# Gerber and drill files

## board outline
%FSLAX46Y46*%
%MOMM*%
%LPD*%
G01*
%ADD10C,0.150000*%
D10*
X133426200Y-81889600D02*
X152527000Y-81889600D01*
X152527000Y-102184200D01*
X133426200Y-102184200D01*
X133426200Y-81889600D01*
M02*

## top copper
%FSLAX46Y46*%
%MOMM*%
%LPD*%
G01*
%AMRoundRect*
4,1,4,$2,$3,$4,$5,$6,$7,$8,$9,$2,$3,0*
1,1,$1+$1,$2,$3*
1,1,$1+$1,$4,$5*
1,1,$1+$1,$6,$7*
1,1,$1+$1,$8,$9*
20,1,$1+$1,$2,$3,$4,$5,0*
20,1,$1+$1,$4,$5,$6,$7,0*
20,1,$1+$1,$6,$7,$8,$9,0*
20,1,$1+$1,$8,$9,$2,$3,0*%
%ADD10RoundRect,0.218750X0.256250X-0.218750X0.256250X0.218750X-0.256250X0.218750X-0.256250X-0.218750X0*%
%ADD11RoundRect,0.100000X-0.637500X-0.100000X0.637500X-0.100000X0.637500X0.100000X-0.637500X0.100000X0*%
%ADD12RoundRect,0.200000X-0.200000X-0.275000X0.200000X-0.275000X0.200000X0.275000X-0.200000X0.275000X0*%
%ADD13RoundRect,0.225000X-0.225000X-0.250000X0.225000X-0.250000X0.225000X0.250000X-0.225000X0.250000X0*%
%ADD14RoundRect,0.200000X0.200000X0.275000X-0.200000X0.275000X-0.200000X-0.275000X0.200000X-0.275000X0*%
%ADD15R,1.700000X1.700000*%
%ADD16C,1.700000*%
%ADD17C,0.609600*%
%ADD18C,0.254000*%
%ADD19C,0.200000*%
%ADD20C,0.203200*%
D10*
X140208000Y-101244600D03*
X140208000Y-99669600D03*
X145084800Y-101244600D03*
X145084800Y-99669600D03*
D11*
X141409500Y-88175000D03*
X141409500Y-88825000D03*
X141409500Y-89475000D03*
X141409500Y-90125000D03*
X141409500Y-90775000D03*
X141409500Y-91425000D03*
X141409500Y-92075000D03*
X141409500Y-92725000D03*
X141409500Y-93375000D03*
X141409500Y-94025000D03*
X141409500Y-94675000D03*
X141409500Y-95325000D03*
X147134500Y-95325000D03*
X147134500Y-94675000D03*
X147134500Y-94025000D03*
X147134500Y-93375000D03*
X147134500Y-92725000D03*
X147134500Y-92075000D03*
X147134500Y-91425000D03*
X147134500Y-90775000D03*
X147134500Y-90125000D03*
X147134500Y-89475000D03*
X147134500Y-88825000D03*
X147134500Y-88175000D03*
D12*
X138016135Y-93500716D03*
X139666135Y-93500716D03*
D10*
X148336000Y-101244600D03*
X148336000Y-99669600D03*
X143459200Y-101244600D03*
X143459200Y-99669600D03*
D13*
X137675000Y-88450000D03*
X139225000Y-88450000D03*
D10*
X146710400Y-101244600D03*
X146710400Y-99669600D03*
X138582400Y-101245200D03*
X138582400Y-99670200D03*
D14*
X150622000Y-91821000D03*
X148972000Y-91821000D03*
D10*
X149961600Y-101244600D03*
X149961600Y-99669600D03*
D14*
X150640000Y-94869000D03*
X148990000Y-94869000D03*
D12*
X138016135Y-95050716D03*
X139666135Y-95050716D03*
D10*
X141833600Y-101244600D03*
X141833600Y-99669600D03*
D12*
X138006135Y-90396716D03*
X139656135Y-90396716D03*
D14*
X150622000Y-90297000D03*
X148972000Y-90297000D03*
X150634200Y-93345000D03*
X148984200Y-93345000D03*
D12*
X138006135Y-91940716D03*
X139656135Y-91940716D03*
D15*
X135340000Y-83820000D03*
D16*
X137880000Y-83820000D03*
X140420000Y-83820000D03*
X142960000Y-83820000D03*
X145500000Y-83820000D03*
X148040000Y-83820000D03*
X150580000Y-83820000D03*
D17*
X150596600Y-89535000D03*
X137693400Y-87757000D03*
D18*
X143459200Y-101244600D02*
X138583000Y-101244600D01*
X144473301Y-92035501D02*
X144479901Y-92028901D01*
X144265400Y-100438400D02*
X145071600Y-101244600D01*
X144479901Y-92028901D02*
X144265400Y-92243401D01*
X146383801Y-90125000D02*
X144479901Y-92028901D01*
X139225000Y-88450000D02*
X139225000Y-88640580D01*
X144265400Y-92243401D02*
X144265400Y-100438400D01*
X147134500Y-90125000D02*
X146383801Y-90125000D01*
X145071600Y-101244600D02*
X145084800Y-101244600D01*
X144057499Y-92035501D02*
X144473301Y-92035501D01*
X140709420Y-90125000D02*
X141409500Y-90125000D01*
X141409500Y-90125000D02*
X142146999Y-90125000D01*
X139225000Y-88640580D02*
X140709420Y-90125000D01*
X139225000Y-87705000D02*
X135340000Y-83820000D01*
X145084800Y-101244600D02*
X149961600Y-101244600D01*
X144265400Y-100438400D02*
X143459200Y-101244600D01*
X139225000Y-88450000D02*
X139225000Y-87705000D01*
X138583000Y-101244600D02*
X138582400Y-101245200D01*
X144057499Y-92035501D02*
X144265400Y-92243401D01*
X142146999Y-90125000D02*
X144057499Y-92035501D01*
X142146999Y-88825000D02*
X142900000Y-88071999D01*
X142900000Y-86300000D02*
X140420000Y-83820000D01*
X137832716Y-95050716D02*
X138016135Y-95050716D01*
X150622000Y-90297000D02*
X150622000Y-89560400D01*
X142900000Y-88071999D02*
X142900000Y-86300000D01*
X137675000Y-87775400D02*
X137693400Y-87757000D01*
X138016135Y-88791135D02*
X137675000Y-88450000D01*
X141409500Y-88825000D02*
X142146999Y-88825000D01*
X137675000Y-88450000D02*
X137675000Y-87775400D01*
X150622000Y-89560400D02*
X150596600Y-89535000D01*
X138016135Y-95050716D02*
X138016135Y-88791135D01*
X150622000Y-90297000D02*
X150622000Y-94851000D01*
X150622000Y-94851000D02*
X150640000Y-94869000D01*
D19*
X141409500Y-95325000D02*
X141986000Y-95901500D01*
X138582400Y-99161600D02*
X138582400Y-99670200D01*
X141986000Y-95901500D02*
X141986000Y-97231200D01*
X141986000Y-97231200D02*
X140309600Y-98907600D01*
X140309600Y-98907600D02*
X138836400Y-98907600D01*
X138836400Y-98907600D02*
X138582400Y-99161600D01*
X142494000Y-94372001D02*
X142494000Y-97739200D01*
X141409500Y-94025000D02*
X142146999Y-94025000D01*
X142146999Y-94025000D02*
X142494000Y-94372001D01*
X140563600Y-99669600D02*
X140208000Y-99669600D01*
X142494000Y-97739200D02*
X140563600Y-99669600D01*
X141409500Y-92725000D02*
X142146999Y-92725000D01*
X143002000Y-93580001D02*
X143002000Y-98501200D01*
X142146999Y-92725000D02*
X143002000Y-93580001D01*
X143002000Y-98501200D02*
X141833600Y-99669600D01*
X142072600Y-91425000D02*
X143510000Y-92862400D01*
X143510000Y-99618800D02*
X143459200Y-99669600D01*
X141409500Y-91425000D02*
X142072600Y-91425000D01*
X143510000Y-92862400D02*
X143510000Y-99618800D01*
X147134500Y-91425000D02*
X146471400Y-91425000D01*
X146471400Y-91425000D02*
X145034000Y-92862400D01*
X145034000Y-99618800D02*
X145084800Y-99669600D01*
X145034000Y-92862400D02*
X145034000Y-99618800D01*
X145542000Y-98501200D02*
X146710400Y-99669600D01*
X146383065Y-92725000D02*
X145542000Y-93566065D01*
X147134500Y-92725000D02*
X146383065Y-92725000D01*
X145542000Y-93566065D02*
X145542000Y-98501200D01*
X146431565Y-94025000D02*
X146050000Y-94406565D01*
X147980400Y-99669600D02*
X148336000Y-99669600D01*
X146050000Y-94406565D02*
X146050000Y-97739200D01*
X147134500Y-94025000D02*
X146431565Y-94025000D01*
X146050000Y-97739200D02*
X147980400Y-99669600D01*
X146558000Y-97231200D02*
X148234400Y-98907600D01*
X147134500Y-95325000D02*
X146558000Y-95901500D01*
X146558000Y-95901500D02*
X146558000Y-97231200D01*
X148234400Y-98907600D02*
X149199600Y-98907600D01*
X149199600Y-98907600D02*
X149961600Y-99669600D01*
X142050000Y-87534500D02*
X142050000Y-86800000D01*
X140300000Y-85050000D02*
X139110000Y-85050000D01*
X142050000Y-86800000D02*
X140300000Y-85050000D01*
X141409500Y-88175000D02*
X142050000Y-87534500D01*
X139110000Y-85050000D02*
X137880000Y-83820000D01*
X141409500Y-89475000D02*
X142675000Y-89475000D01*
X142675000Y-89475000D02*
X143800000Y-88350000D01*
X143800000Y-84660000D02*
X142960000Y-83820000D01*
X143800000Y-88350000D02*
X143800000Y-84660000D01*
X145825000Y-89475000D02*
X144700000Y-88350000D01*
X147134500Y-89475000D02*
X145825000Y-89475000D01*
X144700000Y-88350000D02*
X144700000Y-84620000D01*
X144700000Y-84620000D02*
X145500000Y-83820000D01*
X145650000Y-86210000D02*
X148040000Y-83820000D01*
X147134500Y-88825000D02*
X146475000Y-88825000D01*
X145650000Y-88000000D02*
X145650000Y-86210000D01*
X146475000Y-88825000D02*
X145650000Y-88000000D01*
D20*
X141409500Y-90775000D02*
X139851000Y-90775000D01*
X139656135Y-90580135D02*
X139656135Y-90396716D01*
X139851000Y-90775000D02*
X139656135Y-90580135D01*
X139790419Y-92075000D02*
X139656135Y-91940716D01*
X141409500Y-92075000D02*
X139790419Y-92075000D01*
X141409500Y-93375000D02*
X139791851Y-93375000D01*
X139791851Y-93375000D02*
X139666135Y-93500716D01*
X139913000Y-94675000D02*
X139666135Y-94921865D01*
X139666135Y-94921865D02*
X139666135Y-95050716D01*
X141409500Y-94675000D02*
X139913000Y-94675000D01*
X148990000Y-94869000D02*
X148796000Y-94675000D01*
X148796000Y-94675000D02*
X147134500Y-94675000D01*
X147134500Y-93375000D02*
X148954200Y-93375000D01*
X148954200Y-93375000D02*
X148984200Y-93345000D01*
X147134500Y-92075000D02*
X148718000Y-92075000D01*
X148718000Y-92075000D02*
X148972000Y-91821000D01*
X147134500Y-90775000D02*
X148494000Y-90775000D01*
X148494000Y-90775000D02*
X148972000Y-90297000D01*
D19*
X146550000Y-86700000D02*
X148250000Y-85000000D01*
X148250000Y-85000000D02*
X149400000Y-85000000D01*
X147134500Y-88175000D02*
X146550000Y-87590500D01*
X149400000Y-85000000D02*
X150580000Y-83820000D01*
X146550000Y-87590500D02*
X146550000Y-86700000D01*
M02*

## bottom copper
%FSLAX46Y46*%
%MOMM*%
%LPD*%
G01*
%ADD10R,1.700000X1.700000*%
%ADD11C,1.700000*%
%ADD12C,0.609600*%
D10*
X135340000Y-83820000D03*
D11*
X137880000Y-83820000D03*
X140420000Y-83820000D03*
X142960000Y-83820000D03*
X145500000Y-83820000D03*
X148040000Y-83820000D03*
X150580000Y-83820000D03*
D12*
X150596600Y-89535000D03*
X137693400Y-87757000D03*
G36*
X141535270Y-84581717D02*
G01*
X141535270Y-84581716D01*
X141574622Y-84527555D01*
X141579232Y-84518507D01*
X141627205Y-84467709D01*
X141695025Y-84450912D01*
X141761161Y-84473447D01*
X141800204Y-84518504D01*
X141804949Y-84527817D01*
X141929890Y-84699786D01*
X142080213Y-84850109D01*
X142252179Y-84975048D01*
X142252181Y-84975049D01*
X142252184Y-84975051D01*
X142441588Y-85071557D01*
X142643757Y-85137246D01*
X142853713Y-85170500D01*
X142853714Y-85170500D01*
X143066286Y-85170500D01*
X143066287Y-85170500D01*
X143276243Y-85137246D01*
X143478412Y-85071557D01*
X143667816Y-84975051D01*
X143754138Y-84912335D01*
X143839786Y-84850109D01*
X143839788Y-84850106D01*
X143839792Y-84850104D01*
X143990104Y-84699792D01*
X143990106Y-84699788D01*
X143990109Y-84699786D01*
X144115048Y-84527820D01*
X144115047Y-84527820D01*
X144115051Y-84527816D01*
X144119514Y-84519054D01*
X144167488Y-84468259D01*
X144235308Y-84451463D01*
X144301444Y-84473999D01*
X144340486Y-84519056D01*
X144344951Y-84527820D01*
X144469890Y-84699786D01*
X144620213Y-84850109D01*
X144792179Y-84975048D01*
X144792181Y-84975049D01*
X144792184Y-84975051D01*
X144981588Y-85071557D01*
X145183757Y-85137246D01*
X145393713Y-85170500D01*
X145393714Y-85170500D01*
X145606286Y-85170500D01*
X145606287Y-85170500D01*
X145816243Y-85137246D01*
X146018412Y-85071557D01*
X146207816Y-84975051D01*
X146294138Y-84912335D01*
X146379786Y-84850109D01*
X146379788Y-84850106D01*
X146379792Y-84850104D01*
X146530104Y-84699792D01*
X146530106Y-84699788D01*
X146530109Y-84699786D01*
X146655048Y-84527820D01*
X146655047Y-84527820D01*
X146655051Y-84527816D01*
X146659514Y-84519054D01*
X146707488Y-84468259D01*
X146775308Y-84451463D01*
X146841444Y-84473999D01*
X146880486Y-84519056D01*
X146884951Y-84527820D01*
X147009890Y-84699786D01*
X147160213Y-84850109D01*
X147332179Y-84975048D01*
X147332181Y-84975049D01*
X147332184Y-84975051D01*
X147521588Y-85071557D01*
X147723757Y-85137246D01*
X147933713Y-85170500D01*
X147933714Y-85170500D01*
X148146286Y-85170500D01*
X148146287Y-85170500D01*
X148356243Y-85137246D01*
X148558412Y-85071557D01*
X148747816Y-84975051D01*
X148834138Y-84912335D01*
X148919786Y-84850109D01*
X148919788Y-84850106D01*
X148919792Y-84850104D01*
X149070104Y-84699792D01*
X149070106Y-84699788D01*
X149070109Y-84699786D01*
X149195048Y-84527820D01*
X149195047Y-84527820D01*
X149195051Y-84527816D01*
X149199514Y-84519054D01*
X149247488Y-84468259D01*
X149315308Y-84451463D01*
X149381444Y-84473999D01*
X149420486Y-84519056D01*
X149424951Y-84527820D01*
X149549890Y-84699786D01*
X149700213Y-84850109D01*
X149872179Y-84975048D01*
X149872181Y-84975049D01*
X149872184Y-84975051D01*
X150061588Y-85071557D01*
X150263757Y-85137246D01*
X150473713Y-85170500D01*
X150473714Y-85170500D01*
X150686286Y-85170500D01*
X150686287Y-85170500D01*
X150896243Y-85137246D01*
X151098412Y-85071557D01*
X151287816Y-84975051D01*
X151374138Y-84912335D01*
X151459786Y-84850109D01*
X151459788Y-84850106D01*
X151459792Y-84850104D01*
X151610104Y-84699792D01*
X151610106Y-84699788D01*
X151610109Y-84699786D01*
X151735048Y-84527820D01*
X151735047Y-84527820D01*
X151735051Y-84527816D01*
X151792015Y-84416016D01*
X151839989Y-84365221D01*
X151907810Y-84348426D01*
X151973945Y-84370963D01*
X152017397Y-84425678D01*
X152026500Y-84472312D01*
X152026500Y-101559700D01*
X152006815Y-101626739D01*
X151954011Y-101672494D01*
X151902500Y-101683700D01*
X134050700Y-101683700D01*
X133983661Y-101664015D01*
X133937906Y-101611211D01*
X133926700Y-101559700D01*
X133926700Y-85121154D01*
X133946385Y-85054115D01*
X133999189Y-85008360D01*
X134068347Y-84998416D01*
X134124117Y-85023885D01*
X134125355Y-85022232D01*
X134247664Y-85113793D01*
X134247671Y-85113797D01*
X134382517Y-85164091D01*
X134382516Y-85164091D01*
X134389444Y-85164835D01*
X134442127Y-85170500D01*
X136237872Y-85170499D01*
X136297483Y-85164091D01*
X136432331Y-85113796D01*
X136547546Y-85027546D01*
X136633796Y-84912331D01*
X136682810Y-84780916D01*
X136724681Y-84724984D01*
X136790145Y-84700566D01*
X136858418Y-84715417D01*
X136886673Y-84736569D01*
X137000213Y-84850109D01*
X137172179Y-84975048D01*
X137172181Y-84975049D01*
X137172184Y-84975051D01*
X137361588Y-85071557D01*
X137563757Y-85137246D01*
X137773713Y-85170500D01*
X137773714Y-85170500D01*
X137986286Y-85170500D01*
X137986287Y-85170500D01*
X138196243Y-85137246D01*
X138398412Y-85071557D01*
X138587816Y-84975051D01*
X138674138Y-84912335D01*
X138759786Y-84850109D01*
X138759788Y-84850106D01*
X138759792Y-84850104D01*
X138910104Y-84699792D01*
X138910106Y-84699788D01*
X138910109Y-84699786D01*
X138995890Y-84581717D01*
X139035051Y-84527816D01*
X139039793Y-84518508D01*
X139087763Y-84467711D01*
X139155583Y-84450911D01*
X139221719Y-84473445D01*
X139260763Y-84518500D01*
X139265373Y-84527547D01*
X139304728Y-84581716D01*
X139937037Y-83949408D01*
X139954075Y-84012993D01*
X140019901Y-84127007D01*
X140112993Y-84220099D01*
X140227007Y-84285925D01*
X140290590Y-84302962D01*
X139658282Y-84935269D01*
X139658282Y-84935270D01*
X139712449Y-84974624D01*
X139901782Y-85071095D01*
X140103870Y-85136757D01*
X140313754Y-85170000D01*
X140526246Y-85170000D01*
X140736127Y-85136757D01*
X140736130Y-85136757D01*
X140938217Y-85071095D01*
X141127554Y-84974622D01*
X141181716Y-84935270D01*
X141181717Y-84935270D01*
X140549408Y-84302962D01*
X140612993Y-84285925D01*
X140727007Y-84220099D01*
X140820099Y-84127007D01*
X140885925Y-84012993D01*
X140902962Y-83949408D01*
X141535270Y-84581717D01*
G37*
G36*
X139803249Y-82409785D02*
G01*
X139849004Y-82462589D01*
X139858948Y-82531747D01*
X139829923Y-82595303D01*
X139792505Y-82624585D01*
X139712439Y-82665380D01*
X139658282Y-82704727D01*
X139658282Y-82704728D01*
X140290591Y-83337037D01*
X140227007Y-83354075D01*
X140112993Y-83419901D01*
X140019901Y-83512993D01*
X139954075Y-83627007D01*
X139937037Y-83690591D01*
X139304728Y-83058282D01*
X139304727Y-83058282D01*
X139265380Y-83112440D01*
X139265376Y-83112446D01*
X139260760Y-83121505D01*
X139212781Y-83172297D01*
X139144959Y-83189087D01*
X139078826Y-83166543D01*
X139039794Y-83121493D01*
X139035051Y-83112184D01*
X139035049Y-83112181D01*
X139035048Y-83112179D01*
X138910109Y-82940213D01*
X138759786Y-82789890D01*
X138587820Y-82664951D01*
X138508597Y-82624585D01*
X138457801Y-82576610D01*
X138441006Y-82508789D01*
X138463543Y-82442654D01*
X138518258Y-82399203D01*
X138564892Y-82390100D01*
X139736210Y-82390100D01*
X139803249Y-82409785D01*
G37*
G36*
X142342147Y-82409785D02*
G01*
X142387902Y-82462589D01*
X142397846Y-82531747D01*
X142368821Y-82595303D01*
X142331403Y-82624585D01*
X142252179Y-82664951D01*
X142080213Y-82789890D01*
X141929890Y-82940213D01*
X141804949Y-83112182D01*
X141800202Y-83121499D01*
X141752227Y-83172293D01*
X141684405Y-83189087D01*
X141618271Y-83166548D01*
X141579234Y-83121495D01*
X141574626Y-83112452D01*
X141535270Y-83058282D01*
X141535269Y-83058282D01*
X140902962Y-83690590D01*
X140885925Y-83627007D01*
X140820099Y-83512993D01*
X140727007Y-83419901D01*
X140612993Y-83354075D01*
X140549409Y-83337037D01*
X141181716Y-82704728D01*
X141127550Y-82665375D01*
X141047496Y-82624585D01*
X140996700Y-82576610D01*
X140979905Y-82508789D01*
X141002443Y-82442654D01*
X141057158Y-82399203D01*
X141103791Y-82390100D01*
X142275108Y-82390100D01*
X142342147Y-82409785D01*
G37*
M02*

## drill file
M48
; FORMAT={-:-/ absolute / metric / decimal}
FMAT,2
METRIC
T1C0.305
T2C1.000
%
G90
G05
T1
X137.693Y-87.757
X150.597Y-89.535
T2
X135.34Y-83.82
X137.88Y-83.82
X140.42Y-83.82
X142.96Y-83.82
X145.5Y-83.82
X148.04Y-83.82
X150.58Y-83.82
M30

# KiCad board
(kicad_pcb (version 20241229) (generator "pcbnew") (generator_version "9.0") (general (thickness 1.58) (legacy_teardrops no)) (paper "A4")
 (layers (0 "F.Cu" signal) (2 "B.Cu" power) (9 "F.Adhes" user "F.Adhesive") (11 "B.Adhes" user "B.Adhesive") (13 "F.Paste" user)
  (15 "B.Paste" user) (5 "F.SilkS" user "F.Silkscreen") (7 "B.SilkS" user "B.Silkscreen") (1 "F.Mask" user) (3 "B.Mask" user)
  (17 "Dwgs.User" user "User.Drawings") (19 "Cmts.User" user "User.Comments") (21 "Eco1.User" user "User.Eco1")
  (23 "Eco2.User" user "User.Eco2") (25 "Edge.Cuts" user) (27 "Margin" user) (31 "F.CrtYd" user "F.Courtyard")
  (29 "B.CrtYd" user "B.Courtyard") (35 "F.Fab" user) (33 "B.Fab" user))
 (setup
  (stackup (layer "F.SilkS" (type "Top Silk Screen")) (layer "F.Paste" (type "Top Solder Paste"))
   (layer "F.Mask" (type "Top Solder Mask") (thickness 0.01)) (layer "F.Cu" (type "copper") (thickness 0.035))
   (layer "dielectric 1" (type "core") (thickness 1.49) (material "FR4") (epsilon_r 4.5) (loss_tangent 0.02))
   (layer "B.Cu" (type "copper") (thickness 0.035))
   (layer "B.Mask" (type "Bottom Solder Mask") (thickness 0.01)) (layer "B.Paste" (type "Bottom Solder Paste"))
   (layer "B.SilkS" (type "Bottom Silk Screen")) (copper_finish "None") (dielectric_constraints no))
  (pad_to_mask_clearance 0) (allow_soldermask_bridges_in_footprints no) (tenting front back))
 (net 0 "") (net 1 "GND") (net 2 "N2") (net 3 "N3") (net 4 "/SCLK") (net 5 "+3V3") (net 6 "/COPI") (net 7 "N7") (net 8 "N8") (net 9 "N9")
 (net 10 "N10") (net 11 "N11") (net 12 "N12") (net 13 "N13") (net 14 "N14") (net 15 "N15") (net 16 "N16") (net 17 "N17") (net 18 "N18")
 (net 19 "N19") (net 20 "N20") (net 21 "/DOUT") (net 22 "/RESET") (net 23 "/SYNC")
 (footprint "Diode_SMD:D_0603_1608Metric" (layer "F.Cu") (at 140.208 100.4571 90)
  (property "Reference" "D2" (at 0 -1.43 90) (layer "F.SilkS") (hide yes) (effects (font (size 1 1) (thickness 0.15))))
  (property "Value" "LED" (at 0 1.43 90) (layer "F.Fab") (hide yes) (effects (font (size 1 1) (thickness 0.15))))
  (pad "1" smd roundrect (at -0.7875 0 90) (size 0.875 0.95) (layers "F.Cu" "F.Mask" "F.Paste") (roundrect_rratio 0.25) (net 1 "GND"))
  (pad "2" smd roundrect (at 0.7875 0 90) (size 0.875 0.95) (layers "F.Cu" "F.Mask" "F.Paste") (roundrect_rratio 0.25) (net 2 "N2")))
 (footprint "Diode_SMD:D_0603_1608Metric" (layer "F.Cu") (at 145.0848 100.4571 90)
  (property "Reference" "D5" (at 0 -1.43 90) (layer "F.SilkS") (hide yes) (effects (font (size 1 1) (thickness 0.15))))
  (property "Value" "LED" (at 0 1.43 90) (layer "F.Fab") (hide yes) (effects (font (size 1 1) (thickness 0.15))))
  (pad "1" smd roundrect (at -0.7875 0 90) (size 0.875 0.95) (layers "F.Cu" "F.Mask" "F.Paste") (roundrect_rratio 0.25) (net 1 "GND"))
  (pad "2" smd roundrect (at 0.7875 0 90) (size 0.875 0.95) (layers "F.Cu" "F.Mask" "F.Paste") (roundrect_rratio 0.25) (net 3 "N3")))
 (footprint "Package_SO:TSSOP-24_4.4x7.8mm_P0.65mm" (layer "F.Cu") (at 144.272 91.75)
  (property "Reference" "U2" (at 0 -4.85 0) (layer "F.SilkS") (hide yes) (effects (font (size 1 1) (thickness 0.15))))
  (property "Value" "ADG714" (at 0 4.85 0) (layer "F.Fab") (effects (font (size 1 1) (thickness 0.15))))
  (pad "1" smd roundrect (at -2.8625 -3.575) (size 1.475 0.4) (layers "F.Cu" "F.Mask" "F.Paste") (roundrect_rratio 0.25) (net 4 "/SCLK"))
  (pad "2" smd roundrect (at -2.8625 -2.925) (size 1.475 0.4) (layers "F.Cu" "F.Mask" "F.Paste") (roundrect_rratio 0.25) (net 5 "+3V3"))
  (pad "3" smd roundrect (at -2.8625 -2.275) (size 1.475 0.4) (layers "F.Cu" "F.Mask" "F.Paste") (roundrect_rratio 0.25) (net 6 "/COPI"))
  (pad "4" smd roundrect (at -2.8625 -1.625) (size 1.475 0.4) (layers "F.Cu" "F.Mask" "F.Paste") (roundrect_rratio 0.25) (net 1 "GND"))
  (pad "5" smd roundrect (at -2.8625 -0.975) (size 1.475 0.4) (layers "F.Cu" "F.Mask" "F.Paste") (roundrect_rratio 0.25) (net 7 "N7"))
  (pad "6" smd roundrect (at -2.8625 -0.325) (size 1.475 0.4) (layers "F.Cu" "F.Mask" "F.Paste") (roundrect_rratio 0.25) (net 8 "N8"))
  (pad "7" smd roundrect (at -2.8625 0.325) (size 1.475 0.4) (layers "F.Cu" "F.Mask" "F.Paste") (roundrect_rratio 0.25) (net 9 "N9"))
  (pad "8" smd roundrect (at -2.8625 0.975) (size 1.475 0.4) (layers "F.Cu" "F.Mask" "F.Paste") (roundrect_rratio 0.25) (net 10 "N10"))
  (pad "9" smd roundrect (at -2.8625 1.625) (size 1.475 0.4) (layers "F.Cu" "F.Mask" "F.Paste") (roundrect_rratio 0.25) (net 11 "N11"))
  (pad "10" smd roundrect (at -2.8625 2.275) (size 1.475 0.4) (layers "F.Cu" "F.Mask" "F.Paste") (roundrect_rratio 0.25) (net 2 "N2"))
  (pad "11" smd roundrect (at -2.8625 2.925) (size 1.475 0.4) (layers "F.Cu" "F.Mask" "F.Paste") (roundrect_rratio 0.25) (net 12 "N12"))
  (pad "12" smd roundrect (at -2.8625 3.575) (size 1.475 0.4) (layers "F.Cu" "F.Mask" "F.Paste") (roundrect_rratio 0.25) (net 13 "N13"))
  (pad "13" smd roundrect (at 2.8625 3.575) (size 1.475 0.4) (layers "F.Cu" "F.Mask" "F.Paste") (roundrect_rratio 0.25) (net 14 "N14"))
  (pad "14" smd roundrect (at 2.8625 2.925) (size 1.475 0.4) (layers "F.Cu" "F.Mask" "F.Paste") (roundrect_rratio 0.25) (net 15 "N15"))
  (pad "15" smd roundrect (at 2.8625 2.275) (size 1.475 0.4) (layers "F.Cu" "F.Mask" "F.Paste") (roundrect_rratio 0.25) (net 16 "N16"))
  (pad "16" smd roundrect (at 2.8625 1.625) (size 1.475 0.4) (layers "F.Cu" "F.Mask" "F.Paste") (roundrect_rratio 0.25) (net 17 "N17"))
  (pad "17" smd roundrect (at 2.8625 0.975) (size 1.475 0.4) (layers "F.Cu" "F.Mask" "F.Paste") (roundrect_rratio 0.25) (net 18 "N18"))
  (pad "18" smd roundrect (at 2.8625 0.325) (size 1.475 0.4) (layers "F.Cu" "F.Mask" "F.Paste") (roundrect_rratio 0.25) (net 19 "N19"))
  (pad "19" smd roundrect (at 2.8625 -0.325) (size 1.475 0.4) (layers "F.Cu" "F.Mask" "F.Paste") (roundrect_rratio 0.25) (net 3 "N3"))
  (pad "20" smd roundrect (at 2.8625 -0.975) (size 1.475 0.4) (layers "F.Cu" "F.Mask" "F.Paste") (roundrect_rratio 0.25) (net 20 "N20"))
  (pad "21" smd roundrect (at 2.8625 -1.625) (size 1.475 0.4) (layers "F.Cu" "F.Mask" "F.Paste") (roundrect_rratio 0.25) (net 1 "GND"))
  (pad "22" smd roundrect (at 2.8625 -2.275) (size 1.475 0.4) (layers "F.Cu" "F.Mask" "F.Paste") (roundrect_rratio 0.25) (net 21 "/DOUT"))
  (pad "23" smd roundrect (at 2.8625 -2.925) (size 1.475 0.4) (layers "F.Cu" "F.Mask" "F.Paste") (roundrect_rratio 0.25) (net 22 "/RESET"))
  (pad "24" smd roundrect (at 2.8625 -3.575) (size 1.475 0.4) (layers "F.Cu" "F.Mask" "F.Paste") (roundrect_rratio 0.25) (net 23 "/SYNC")))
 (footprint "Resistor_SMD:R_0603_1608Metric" (layer "F.Cu") (at 138.841135 93.500716)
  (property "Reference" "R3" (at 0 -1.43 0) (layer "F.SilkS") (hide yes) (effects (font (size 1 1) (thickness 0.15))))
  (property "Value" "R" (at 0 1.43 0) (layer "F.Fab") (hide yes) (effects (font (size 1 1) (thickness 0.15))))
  (pad "1" smd roundrect (at -0.825 0) (size 0.8 0.95) (layers "F.Cu" "F.Mask" "F.Paste") (roundrect_rratio 0.25) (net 5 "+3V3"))
  (pad "2" smd roundrect (at 0.825 0) (size 0.8 0.95) (layers "F.Cu" "F.Mask" "F.Paste") (roundrect_rratio 0.25) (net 11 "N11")))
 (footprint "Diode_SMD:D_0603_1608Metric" (layer "F.Cu") (at 148.336 100.4571 90)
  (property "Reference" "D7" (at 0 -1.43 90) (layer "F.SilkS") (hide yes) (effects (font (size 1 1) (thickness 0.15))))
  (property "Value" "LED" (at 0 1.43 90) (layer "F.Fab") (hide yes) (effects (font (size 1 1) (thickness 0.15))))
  (pad "1" smd roundrect (at -0.7875 0 90) (size 0.875 0.95) (layers "F.Cu" "F.Mask" "F.Paste") (roundrect_rratio 0.25) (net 1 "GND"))
  (pad "2" smd roundrect (at 0.7875 0 90) (size 0.875 0.95) (layers "F.Cu" "F.Mask" "F.Paste") (roundrect_rratio 0.25) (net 16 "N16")))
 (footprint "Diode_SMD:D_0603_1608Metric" (layer "F.Cu") (at 143.4592 100.4571 90)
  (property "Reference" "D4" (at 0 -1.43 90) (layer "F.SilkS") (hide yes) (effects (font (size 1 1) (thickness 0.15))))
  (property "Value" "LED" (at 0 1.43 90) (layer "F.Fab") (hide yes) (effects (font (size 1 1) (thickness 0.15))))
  (pad "1" smd roundrect (at -0.7875 0 90) (size 0.875 0.95) (layers "F.Cu" "F.Mask" "F.Paste") (roundrect_rratio 0.25) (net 1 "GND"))
  (pad "2" smd roundrect (at 0.7875 0 90) (size 0.875 0.95) (layers "F.Cu" "F.Mask" "F.Paste") (roundrect_rratio 0.25) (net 8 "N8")))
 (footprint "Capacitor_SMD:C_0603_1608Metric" (layer "F.Cu") (at 138.45 88.45)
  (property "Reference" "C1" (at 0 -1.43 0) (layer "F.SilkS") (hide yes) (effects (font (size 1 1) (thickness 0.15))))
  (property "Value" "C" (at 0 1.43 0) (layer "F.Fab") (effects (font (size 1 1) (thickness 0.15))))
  (pad "1" smd roundrect (at -0.775 0) (size 0.9 0.95) (layers "F.Cu" "F.Mask" "F.Paste") (roundrect_rratio 0.25) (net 5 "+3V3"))
  (pad "2" smd roundrect (at 0.775 0) (size 0.9 0.95) (layers "F.Cu" "F.Mask" "F.Paste") (roundrect_rratio 0.25) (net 1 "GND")))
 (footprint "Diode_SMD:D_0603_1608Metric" (layer "F.Cu") (at 146.7104 100.4571 90)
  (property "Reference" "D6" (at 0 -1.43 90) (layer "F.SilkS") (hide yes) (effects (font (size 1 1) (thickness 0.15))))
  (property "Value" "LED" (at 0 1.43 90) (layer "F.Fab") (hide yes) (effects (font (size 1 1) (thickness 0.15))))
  (pad "1" smd roundrect (at -0.7875 0 90) (size 0.875 0.95) (layers "F.Cu" "F.Mask" "F.Paste") (roundrect_rratio 0.25) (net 1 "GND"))
  (pad "2" smd roundrect (at 0.7875 0 90) (size 0.875 0.95) (layers "F.Cu" "F.Mask" "F.Paste") (roundrect_rratio 0.25) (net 18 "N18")))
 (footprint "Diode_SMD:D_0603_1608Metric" (layer "F.Cu") (at 138.5824 100.4577 90)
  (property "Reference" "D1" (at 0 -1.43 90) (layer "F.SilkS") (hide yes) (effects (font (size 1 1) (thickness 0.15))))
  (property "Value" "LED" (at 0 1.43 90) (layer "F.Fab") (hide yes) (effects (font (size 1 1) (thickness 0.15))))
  (pad "1" smd roundrect (at -0.7875 0 90) (size 0.875 0.95) (layers "F.Cu" "F.Mask" "F.Paste") (roundrect_rratio 0.25) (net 1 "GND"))
  (pad "2" smd roundrect (at 0.7875 0 90) (size 0.875 0.95) (layers "F.Cu" "F.Mask" "F.Paste") (roundrect_rratio 0.25) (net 13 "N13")))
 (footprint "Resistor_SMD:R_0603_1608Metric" (layer "F.Cu") (at 149.797 91.821 180)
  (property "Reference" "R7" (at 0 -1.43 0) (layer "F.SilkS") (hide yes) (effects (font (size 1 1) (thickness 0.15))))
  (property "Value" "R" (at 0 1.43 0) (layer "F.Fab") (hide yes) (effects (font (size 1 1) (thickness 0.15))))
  (pad "1" smd roundrect (at -0.825 0 180) (size 0.8 0.95) (layers "F.Cu" "F.Mask" "F.Paste") (roundrect_rratio 0.25) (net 5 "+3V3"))
  (pad "2" smd roundrect (at 0.825 0 180) (size 0.8 0.95) (layers "F.Cu" "F.Mask" "F.Paste") (roundrect_rratio 0.25) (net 19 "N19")))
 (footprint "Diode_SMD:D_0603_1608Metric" (layer "F.Cu") (at 149.9616 100.4571 90)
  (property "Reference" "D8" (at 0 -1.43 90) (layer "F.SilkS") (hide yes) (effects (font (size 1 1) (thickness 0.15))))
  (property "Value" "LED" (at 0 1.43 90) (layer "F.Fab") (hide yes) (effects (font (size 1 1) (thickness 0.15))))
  (pad "1" smd roundrect (at -0.7875 0 90) (size 0.875 0.95) (layers "F.Cu" "F.Mask" "F.Paste") (roundrect_rratio 0.25) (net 1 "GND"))
  (pad "2" smd roundrect (at 0.7875 0 90) (size 0.875 0.95) (layers "F.Cu" "F.Mask" "F.Paste") (roundrect_rratio 0.25) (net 14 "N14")))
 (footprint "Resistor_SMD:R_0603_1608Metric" (layer "F.Cu") (at 149.815 94.869 180)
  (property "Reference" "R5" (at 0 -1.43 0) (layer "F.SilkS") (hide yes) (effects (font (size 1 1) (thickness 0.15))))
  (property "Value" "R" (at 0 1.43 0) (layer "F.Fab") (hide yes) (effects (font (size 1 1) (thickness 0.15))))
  (pad "1" smd roundrect (at -0.825 0 180) (size 0.8 0.95) (layers "F.Cu" "F.Mask" "F.Paste") (roundrect_rratio 0.25) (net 5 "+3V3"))
  (pad "2" smd roundrect (at 0.825 0 180) (size 0.8 0.95) (layers "F.Cu" "F.Mask" "F.Paste") (roundrect_rratio 0.25) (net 15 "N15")))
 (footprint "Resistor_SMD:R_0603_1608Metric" (layer "F.Cu") (at 138.841135 95.050716)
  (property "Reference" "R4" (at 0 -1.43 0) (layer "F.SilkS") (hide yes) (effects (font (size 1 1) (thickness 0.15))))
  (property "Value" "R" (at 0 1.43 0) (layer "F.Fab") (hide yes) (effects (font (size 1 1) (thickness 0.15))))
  (pad "1" smd roundrect (at -0.825 0) (size 0.8 0.95) (layers "F.Cu" "F.Mask" "F.Paste") (roundrect_rratio 0.25) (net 5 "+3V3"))
  (pad "2" smd roundrect (at 0.825 0) (size 0.8 0.95) (layers "F.Cu" "F.Mask" "F.Paste") (roundrect_rratio 0.25) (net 12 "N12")))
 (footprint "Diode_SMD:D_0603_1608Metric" (layer "F.Cu") (at 141.8336 100.4571 90)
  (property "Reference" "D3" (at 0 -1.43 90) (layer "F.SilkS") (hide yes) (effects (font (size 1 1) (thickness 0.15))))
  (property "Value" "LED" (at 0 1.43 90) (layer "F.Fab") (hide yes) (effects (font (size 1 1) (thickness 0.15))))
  (pad "1" smd roundrect (at -0.7875 0 90) (size 0.875 0.95) (layers "F.Cu" "F.Mask" "F.Paste") (roundrect_rratio 0.25) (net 1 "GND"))
  (pad "2" smd roundrect (at 0.7875 0 90) (size 0.875 0.95) (layers "F.Cu" "F.Mask" "F.Paste") (roundrect_rratio 0.25) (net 10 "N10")))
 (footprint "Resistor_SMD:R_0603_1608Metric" (layer "F.Cu") (at 138.831135 90.396716)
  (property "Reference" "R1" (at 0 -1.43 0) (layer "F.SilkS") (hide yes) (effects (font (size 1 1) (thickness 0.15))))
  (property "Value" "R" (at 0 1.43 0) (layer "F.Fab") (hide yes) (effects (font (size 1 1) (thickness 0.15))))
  (pad "1" smd roundrect (at -0.825 0) (size 0.8 0.95) (layers "F.Cu" "F.Mask" "F.Paste") (roundrect_rratio 0.25) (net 5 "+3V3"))
  (pad "2" smd roundrect (at 0.825 0) (size 0.8 0.95) (layers "F.Cu" "F.Mask" "F.Paste") (roundrect_rratio 0.25) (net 7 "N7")))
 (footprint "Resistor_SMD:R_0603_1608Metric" (layer "F.Cu") (at 149.797 90.297 180)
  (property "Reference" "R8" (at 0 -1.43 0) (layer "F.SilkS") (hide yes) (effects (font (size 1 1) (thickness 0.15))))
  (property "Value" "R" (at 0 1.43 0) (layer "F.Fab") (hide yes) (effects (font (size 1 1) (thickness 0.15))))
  (pad "1" smd roundrect (at -0.825 0 180) (size 0.8 0.95) (layers "F.Cu" "F.Mask" "F.Paste") (roundrect_rratio 0.25) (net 5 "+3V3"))
  (pad "2" smd roundrect (at 0.825 0 180) (size 0.8 0.95) (layers "F.Cu" "F.Mask" "F.Paste") (roundrect_rratio 0.25) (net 20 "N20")))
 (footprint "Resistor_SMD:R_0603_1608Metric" (layer "F.Cu") (at 149.8092 93.345 180)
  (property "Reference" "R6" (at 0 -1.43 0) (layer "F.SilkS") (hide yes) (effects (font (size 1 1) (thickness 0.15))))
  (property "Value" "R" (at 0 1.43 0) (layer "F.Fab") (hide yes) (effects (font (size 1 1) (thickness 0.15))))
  (pad "1" smd roundrect (at -0.825 0 180) (size 0.8 0.95) (layers "F.Cu" "F.Mask" "F.Paste") (roundrect_rratio 0.25) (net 5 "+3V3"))
  (pad "2" smd roundrect (at 0.825 0 180) (size 0.8 0.95) (layers "F.Cu" "F.Mask" "F.Paste") (roundrect_rratio 0.25) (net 17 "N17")))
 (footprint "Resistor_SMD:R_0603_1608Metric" (layer "F.Cu") (at 138.831135 91.940716)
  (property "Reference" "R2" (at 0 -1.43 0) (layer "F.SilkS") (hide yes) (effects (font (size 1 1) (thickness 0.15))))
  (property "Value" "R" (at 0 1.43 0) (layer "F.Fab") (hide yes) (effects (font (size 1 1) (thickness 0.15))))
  (pad "1" smd roundrect (at -0.825 0) (size 0.8 0.95) (layers "F.Cu" "F.Mask" "F.Paste") (roundrect_rratio 0.25) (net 5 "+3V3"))
  (pad "2" smd roundrect (at 0.825 0) (size 0.8 0.95) (layers "F.Cu" "F.Mask" "F.Paste") (roundrect_rratio 0.25) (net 9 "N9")))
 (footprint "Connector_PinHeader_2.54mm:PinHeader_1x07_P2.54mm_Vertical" (layer "B.Cu") (at 135.34 83.82 -90)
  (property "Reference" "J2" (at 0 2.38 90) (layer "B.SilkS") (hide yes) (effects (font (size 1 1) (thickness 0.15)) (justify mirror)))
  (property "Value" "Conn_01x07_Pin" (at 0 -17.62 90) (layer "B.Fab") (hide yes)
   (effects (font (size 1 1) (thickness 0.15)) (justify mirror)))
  (pad "1" thru_hole rect (at 0 0 270) (size 1.7 1.7) (drill 1) (layers "*.Cu" "*.Mask") (remove_unused_layers no) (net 1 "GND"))
  (pad "2" thru_hole circle (at 0 -2.54 270) (size 1.7 1.7) (drill 1) (layers "*.Cu" "*.Mask") (remove_unused_layers no) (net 4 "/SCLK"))
  (pad "3" thru_hole circle (at 0 -5.08 270) (size 1.7 1.7) (drill 1) (layers "*.Cu" "*.Mask") (remove_unused_layers no) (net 5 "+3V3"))
  (pad "4" thru_hole circle (at 0 -7.62 270) (size 1.7 1.7) (drill 1) (layers "*.Cu" "*.Mask") (remove_unused_layers no) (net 6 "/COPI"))
  (pad "5" thru_hole circle (at 0 -10.16 270) (size 1.7 1.7) (drill 1) (layers "*.Cu" "*.Mask") (remove_unused_layers no) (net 21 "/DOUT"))
  (pad "6" thru_hole circle (at 0 -12.7 270) (size 1.7 1.7) (drill 1) (layers "*.Cu" "*.Mask") (remove_unused_layers no) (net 22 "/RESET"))
  (pad "7" thru_hole circle (at 0 -15.24 270) (size 1.7 1.7) (drill 1) (layers "*.Cu" "*.Mask") (remove_unused_layers no) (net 23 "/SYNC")))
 (gr_rect (start 133.4262 81.8896) (end 152.527 102.1842) (stroke (width 0.15) (type default)) (fill no) (layer "Edge.Cuts"))
 (segment (start 143.4592 101.2446) (end 138.583 101.2446) (width 0.254) (layer "F.Cu") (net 1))
 (segment (start 144.473301 92.035501) (end 144.479901 92.028901) (width 0.254) (layer "F.Cu") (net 1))
 (segment (start 144.2654 100.4384) (end 145.0716 101.2446) (width 0.254) (layer "F.Cu") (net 1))
 (segment (start 144.479901 92.028901) (end 144.2654 92.243401) (width 0.254) (layer "F.Cu") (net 1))
 (segment (start 146.383801 90.125) (end 144.479901 92.028901) (width 0.254) (layer "F.Cu") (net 1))
 (segment (start 139.225 88.45) (end 139.225 88.64058) (width 0.254) (layer "F.Cu") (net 1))
 (segment (start 144.2654 92.243401) (end 144.2654 100.4384) (width 0.254) (layer "F.Cu") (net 1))
 (segment (start 147.1345 90.125) (end 146.383801 90.125) (width 0.254) (layer "F.Cu") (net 1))
 (segment (start 145.0716 101.2446) (end 145.0848 101.2446) (width 0.254) (layer "F.Cu") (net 1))
 (segment (start 144.057499 92.035501) (end 144.473301 92.035501) (width 0.254) (layer "F.Cu") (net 1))
 (segment (start 140.70942 90.125) (end 141.4095 90.125) (width 0.254) (layer "F.Cu") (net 1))
 (segment (start 141.4095 90.125) (end 142.146999 90.125) (width 0.254) (layer "F.Cu") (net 1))
 (segment (start 139.225 88.64058) (end 140.70942 90.125) (width 0.254) (layer "F.Cu") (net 1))
 (segment (start 139.225 87.705) (end 135.34 83.82) (width 0.254) (layer "F.Cu") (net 1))
 (segment (start 145.0848 101.2446) (end 149.9616 101.2446) (width 0.254) (layer "F.Cu") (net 1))
 (segment (start 144.2654 100.4384) (end 143.4592 101.2446) (width 0.254) (layer "F.Cu") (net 1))
 (segment (start 139.225 88.45) (end 139.225 87.705) (width 0.254) (layer "F.Cu") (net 1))
 (segment (start 138.583 101.2446) (end 138.5824 101.2452) (width 0.254) (layer "F.Cu") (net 1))
 (segment (start 144.057499 92.035501) (end 144.2654 92.243401) (width 0.254) (layer "F.Cu") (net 1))
 (segment (start 142.146999 90.125) (end 144.057499 92.035501) (width 0.254) (layer "F.Cu") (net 1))
 (segment (start 142.146999 88.825) (end 142.9 88.071999) (width 0.254) (layer "F.Cu") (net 5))
 (segment (start 142.9 86.3) (end 140.42 83.82) (width 0.254) (layer "F.Cu") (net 5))
 (segment (start 137.832716 95.050716) (end 138.016135 95.050716) (width 0.254) (layer "F.Cu") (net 5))
 (segment (start 150.622 90.297) (end 150.622 89.5604) (width 0.254) (layer "F.Cu") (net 5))
 (segment (start 142.9 88.071999) (end 142.9 86.3) (width 0.254) (layer "F.Cu") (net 5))
 (segment (start 137.675 87.7754) (end 137.6934 87.757) (width 0.254) (layer "F.Cu") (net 5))
 (segment (start 138.016135 88.791135) (end 137.675 88.45) (width 0.254) (layer "F.Cu") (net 5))
 (segment (start 141.4095 88.825) (end 142.146999 88.825) (width 0.254) (layer "F.Cu") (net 5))
 (segment (start 137.675 88.45) (end 137.675 87.7754) (width 0.254) (layer "F.Cu") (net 5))
 (segment (start 150.622 89.5604) (end 150.5966 89.535) (width 0.254) (layer "F.Cu") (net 5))
 (segment (start 138.016135 95.050716) (end 138.016135 88.791135) (width 0.254) (layer "F.Cu") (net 5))
 (segment (start 150.622 90.297) (end 150.622 94.851) (width 0.254) (layer "F.Cu") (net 5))
 (segment (start 150.622 94.851) (end 150.64 94.869) (width 0.254) (layer "F.Cu") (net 5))
 (via (at 150.5966 89.535) (size 0.6096) (drill 0.3048) (layers "F.Cu" "B.Cu") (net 5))
 (via (at 137.6934 87.757) (size 0.6096) (drill 0.3048) (layers "F.Cu" "B.Cu") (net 5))
 (segment (start 141.4095 95.325) (end 141.986 95.9015) (width 0.2) (layer "F.Cu") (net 13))
 (segment (start 138.5824 99.1616) (end 138.5824 99.6702) (width 0.2) (layer "F.Cu") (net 13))
 (segment (start 141.986 95.9015) (end 141.986 97.2312) (width 0.2) (layer "F.Cu") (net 13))
 (segment (start 141.986 97.2312) (end 140.3096 98.9076) (width 0.2) (layer "F.Cu") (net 13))
 (segment (start 140.3096 98.9076) (end 138.8364 98.9076) (width 0.2) (layer "F.Cu") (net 13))
 (segment (start 138.8364 98.9076) (end 138.5824 99.1616) (width 0.2) (layer "F.Cu") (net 13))
 (segment (start 142.494 94.372001) (end 142.494 97.7392) (width 0.2) (layer "F.Cu") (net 2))
 (segment (start 141.4095 94.025) (end 142.146999 94.025) (width 0.2) (layer "F.Cu") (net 2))
 (segment (start 142.146999 94.025) (end 142.494 94.372001) (width 0.2) (layer "F.Cu") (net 2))
 (segment (start 140.5636 99.6696) (end 140.208 99.6696) (width 0.2) (layer "F.Cu") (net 2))
 (segment (start 142.494 97.7392) (end 140.5636 99.6696) (width 0.2) (layer "F.Cu") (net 2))
 (segment (start 141.4095 92.725) (end 142.146999 92.725) (width 0.2) (layer "F.Cu") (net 10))
 (segment (start 143.002 93.580001) (end 143.002 98.5012) (width 0.2) (layer "F.Cu") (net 10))
 (segment (start 142.146999 92.725) (end 143.002 93.580001) (width 0.2) (layer "F.Cu") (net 10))
 (segment (start 143.002 98.5012) (end 141.8336 99.6696) (width 0.2) (layer "F.Cu") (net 10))
 (segment (start 142.0726 91.425) (end 143.51 92.8624) (width 0.2) (layer "F.Cu") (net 8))
 (segment (start 143.51 99.6188) (end 143.4592 99.6696) (width 0.2) (layer "F.Cu") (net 8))
 (segment (start 141.4095 91.425) (end 142.0726 91.425) (width 0.2) (layer "F.Cu") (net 8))
 (segment (start 143.51 92.8624) (end 143.51 99.6188) (width 0.2) (layer "F.Cu") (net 8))
 (segment (start 147.1345 91.425) (end 146.4714 91.425) (width 0.2) (layer "F.Cu") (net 3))
 (segment (start 146.4714 91.425) (end 145.034 92.8624) (width 0.2) (layer "F.Cu") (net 3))
 (segment (start 145.034 99.6188) (end 145.0848 99.6696) (width 0.2) (layer "F.Cu") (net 3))
 (segment (start 145.034 92.8624) (end 145.034 99.6188) (width 0.2) (layer "F.Cu") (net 3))
 (segment (start 145.542 98.5012) (end 146.7104 99.6696) (width 0.2) (layer "F.Cu") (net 18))
 (segment (start 146.383065 92.725) (end 145.542 93.566065) (width 0.2) (layer "F.Cu") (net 18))
 (segment (start 147.1345 92.725) (end 146.383065 92.725) (width 0.2) (layer "F.Cu") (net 18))
 (segment (start 145.542 93.566065) (end 145.542 98.5012) (width 0.2) (layer "F.Cu") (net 18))
 (segment (start 146.431565 94.025) (end 146.05 94.406565) (width 0.2) (layer "F.Cu") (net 16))
 (segment (start 147.9804 99.6696) (end 148.336 99.6696) (width 0.2) (layer "F.Cu") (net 16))
 (segment (start 146.05 94.406565) (end 146.05 97.7392) (width 0.2) (layer "F.Cu") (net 16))
 (segment (start 147.1345 94.025) (end 146.431565 94.025) (width 0.2) (layer "F.Cu") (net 16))
 (segment (start 146.05 97.7392) (end 147.9804 99.6696) (width 0.2) (layer "F.Cu") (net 16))
 (segment (start 146.558 97.2312) (end 148.2344 98.9076) (width 0.2) (layer "F.Cu") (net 14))
 (segment (start 147.1345 95.325) (end 146.558 95.9015) (width 0.2) (layer "F.Cu") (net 14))
 (segment (start 146.558 95.9015) (end 146.558 97.2312) (width 0.2) (layer "F.Cu") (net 14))
 (segment (start 148.2344 98.9076) (end 149.1996 98.9076) (width 0.2) (layer "F.Cu") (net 14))
 (segment (start 149.1996 98.9076) (end 149.9616 99.6696) (width 0.2) (layer "F.Cu") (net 14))
 (segment (start 142.05 87.5345) (end 142.05 86.8) (width 0.2) (layer "F.Cu") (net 4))
 (segment (start 140.3 85.05) (end 139.11 85.05) (width 0.2) (layer "F.Cu") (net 4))
 (segment (start 142.05 86.8) (end 140.3 85.05) (width 0.2) (layer "F.Cu") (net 4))
 (segment (start 141.4095 88.175) (end 142.05 87.5345) (width 0.2) (layer "F.Cu") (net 4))
 (segment (start 139.11 85.05) (end 137.88 83.82) (width 0.2) (layer "F.Cu") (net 4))
 (segment (start 141.4095 89.475) (end 142.675 89.475) (width 0.2) (layer "F.Cu") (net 6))
 (segment (start 142.675 89.475) (end 143.8 88.35) (width 0.2) (layer "F.Cu") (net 6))
 (segment (start 143.8 84.66) (end 142.96 83.82) (width 0.2) (layer "F.Cu") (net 6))
 (segment (start 143.8 88.35) (end 143.8 84.66) (width 0.2) (layer "F.Cu") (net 6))
 (segment (start 145.825 89.475) (end 144.7 88.35) (width 0.2) (layer "F.Cu") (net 21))
 (segment (start 147.1345 89.475) (end 145.825 89.475) (width 0.2) (layer "F.Cu") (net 21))
 (segment (start 144.7 88.35) (end 144.7 84.62) (width 0.2) (layer "F.Cu") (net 21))
 (segment (start 144.7 84.62) (end 145.5 83.82) (width 0.2) (layer "F.Cu") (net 21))
 (segment (start 145.65 86.21) (end 148.04 83.82) (width 0.2) (layer "F.Cu") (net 22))
 (segment (start 147.1345 88.825) (end 146.475 88.825) (width 0.2) (layer "F.Cu") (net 22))
 (segment (start 145.65 88) (end 145.65 86.21) (width 0.2) (layer "F.Cu") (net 22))
 (segment (start 146.475 88.825) (end 145.65 88) (width 0.2) (layer "F.Cu") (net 22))
 (segment (start 141.4095 90.775) (end 139.851 90.775) (width 0.2032) (layer "F.Cu") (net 7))
 (segment (start 139.656135 90.580135) (end 139.656135 90.396716) (width 0.2032) (layer "F.Cu") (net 7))
 (segment (start 139.851 90.775) (end 139.656135 90.580135) (width 0.2032) (layer "F.Cu") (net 7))
 (segment (start 139.790419 92.075) (end 139.656135 91.940716) (width 0.2032) (layer "F.Cu") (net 9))
 (segment (start 141.4095 92.075) (end 139.790419 92.075) (width 0.2032) (layer "F.Cu") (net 9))
 (segment (start 141.4095 93.375) (end 139.791851 93.375) (width 0.2032) (layer "F.Cu") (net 11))
 (segment (start 139.791851 93.375) (end 139.666135 93.500716) (width 0.2032) (layer "F.Cu") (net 11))
 (segment (start 139.913 94.675) (end 139.666135 94.921865) (width 0.2032) (layer "F.Cu") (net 12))
 (segment (start 139.666135 94.921865) (end 139.666135 95.050716) (width 0.2032) (layer "F.Cu") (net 12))
 (segment (start 141.4095 94.675) (end 139.913 94.675) (width 0.2032) (layer "F.Cu") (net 12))
 (segment (start 148.99 94.869) (end 148.796 94.675) (width 0.2032) (layer "F.Cu") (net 15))
 (segment (start 148.796 94.675) (end 147.1345 94.675) (width 0.2032) (layer "F.Cu") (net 15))
 (segment (start 147.1345 93.375) (end 148.9542 93.375) (width 0.2032) (layer "F.Cu") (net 17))
 (segment (start 148.9542 93.375) (end 148.9842 93.345) (width 0.2032) (layer "F.Cu") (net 17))
 (segment (start 147.1345 92.075) (end 148.718 92.075) (width 0.2032) (layer "F.Cu") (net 19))
 (segment (start 148.718 92.075) (end 148.972 91.821) (width 0.2032) (layer "F.Cu") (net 19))
 (segment (start 147.1345 90.775) (end 148.494 90.775) (width 0.2032) (layer "F.Cu") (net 20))
 (segment (start 148.494 90.775) (end 148.972 90.297) (width 0.2032) (layer "F.Cu") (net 20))
 (segment (start 146.55 86.7) (end 148.25 85) (width 0.2) (layer "F.Cu") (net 23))
 (segment (start 148.25 85) (end 149.4 85) (width 0.2) (layer "F.Cu") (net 23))
 (segment (start 147.1345 88.175) (end 146.55 87.5905) (width 0.2) (layer "F.Cu") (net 23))
 (segment (start 149.4 85) (end 150.58 83.82) (width 0.2) (layer "F.Cu") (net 23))
 (segment (start 146.55 87.5905) (end 146.55 86.7) (width 0.2) (layer "F.Cu") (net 23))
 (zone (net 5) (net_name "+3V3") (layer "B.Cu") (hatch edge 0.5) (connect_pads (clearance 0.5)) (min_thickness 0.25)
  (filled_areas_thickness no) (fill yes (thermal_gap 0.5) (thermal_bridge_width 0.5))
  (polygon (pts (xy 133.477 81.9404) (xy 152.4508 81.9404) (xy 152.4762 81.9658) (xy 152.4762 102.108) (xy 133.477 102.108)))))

